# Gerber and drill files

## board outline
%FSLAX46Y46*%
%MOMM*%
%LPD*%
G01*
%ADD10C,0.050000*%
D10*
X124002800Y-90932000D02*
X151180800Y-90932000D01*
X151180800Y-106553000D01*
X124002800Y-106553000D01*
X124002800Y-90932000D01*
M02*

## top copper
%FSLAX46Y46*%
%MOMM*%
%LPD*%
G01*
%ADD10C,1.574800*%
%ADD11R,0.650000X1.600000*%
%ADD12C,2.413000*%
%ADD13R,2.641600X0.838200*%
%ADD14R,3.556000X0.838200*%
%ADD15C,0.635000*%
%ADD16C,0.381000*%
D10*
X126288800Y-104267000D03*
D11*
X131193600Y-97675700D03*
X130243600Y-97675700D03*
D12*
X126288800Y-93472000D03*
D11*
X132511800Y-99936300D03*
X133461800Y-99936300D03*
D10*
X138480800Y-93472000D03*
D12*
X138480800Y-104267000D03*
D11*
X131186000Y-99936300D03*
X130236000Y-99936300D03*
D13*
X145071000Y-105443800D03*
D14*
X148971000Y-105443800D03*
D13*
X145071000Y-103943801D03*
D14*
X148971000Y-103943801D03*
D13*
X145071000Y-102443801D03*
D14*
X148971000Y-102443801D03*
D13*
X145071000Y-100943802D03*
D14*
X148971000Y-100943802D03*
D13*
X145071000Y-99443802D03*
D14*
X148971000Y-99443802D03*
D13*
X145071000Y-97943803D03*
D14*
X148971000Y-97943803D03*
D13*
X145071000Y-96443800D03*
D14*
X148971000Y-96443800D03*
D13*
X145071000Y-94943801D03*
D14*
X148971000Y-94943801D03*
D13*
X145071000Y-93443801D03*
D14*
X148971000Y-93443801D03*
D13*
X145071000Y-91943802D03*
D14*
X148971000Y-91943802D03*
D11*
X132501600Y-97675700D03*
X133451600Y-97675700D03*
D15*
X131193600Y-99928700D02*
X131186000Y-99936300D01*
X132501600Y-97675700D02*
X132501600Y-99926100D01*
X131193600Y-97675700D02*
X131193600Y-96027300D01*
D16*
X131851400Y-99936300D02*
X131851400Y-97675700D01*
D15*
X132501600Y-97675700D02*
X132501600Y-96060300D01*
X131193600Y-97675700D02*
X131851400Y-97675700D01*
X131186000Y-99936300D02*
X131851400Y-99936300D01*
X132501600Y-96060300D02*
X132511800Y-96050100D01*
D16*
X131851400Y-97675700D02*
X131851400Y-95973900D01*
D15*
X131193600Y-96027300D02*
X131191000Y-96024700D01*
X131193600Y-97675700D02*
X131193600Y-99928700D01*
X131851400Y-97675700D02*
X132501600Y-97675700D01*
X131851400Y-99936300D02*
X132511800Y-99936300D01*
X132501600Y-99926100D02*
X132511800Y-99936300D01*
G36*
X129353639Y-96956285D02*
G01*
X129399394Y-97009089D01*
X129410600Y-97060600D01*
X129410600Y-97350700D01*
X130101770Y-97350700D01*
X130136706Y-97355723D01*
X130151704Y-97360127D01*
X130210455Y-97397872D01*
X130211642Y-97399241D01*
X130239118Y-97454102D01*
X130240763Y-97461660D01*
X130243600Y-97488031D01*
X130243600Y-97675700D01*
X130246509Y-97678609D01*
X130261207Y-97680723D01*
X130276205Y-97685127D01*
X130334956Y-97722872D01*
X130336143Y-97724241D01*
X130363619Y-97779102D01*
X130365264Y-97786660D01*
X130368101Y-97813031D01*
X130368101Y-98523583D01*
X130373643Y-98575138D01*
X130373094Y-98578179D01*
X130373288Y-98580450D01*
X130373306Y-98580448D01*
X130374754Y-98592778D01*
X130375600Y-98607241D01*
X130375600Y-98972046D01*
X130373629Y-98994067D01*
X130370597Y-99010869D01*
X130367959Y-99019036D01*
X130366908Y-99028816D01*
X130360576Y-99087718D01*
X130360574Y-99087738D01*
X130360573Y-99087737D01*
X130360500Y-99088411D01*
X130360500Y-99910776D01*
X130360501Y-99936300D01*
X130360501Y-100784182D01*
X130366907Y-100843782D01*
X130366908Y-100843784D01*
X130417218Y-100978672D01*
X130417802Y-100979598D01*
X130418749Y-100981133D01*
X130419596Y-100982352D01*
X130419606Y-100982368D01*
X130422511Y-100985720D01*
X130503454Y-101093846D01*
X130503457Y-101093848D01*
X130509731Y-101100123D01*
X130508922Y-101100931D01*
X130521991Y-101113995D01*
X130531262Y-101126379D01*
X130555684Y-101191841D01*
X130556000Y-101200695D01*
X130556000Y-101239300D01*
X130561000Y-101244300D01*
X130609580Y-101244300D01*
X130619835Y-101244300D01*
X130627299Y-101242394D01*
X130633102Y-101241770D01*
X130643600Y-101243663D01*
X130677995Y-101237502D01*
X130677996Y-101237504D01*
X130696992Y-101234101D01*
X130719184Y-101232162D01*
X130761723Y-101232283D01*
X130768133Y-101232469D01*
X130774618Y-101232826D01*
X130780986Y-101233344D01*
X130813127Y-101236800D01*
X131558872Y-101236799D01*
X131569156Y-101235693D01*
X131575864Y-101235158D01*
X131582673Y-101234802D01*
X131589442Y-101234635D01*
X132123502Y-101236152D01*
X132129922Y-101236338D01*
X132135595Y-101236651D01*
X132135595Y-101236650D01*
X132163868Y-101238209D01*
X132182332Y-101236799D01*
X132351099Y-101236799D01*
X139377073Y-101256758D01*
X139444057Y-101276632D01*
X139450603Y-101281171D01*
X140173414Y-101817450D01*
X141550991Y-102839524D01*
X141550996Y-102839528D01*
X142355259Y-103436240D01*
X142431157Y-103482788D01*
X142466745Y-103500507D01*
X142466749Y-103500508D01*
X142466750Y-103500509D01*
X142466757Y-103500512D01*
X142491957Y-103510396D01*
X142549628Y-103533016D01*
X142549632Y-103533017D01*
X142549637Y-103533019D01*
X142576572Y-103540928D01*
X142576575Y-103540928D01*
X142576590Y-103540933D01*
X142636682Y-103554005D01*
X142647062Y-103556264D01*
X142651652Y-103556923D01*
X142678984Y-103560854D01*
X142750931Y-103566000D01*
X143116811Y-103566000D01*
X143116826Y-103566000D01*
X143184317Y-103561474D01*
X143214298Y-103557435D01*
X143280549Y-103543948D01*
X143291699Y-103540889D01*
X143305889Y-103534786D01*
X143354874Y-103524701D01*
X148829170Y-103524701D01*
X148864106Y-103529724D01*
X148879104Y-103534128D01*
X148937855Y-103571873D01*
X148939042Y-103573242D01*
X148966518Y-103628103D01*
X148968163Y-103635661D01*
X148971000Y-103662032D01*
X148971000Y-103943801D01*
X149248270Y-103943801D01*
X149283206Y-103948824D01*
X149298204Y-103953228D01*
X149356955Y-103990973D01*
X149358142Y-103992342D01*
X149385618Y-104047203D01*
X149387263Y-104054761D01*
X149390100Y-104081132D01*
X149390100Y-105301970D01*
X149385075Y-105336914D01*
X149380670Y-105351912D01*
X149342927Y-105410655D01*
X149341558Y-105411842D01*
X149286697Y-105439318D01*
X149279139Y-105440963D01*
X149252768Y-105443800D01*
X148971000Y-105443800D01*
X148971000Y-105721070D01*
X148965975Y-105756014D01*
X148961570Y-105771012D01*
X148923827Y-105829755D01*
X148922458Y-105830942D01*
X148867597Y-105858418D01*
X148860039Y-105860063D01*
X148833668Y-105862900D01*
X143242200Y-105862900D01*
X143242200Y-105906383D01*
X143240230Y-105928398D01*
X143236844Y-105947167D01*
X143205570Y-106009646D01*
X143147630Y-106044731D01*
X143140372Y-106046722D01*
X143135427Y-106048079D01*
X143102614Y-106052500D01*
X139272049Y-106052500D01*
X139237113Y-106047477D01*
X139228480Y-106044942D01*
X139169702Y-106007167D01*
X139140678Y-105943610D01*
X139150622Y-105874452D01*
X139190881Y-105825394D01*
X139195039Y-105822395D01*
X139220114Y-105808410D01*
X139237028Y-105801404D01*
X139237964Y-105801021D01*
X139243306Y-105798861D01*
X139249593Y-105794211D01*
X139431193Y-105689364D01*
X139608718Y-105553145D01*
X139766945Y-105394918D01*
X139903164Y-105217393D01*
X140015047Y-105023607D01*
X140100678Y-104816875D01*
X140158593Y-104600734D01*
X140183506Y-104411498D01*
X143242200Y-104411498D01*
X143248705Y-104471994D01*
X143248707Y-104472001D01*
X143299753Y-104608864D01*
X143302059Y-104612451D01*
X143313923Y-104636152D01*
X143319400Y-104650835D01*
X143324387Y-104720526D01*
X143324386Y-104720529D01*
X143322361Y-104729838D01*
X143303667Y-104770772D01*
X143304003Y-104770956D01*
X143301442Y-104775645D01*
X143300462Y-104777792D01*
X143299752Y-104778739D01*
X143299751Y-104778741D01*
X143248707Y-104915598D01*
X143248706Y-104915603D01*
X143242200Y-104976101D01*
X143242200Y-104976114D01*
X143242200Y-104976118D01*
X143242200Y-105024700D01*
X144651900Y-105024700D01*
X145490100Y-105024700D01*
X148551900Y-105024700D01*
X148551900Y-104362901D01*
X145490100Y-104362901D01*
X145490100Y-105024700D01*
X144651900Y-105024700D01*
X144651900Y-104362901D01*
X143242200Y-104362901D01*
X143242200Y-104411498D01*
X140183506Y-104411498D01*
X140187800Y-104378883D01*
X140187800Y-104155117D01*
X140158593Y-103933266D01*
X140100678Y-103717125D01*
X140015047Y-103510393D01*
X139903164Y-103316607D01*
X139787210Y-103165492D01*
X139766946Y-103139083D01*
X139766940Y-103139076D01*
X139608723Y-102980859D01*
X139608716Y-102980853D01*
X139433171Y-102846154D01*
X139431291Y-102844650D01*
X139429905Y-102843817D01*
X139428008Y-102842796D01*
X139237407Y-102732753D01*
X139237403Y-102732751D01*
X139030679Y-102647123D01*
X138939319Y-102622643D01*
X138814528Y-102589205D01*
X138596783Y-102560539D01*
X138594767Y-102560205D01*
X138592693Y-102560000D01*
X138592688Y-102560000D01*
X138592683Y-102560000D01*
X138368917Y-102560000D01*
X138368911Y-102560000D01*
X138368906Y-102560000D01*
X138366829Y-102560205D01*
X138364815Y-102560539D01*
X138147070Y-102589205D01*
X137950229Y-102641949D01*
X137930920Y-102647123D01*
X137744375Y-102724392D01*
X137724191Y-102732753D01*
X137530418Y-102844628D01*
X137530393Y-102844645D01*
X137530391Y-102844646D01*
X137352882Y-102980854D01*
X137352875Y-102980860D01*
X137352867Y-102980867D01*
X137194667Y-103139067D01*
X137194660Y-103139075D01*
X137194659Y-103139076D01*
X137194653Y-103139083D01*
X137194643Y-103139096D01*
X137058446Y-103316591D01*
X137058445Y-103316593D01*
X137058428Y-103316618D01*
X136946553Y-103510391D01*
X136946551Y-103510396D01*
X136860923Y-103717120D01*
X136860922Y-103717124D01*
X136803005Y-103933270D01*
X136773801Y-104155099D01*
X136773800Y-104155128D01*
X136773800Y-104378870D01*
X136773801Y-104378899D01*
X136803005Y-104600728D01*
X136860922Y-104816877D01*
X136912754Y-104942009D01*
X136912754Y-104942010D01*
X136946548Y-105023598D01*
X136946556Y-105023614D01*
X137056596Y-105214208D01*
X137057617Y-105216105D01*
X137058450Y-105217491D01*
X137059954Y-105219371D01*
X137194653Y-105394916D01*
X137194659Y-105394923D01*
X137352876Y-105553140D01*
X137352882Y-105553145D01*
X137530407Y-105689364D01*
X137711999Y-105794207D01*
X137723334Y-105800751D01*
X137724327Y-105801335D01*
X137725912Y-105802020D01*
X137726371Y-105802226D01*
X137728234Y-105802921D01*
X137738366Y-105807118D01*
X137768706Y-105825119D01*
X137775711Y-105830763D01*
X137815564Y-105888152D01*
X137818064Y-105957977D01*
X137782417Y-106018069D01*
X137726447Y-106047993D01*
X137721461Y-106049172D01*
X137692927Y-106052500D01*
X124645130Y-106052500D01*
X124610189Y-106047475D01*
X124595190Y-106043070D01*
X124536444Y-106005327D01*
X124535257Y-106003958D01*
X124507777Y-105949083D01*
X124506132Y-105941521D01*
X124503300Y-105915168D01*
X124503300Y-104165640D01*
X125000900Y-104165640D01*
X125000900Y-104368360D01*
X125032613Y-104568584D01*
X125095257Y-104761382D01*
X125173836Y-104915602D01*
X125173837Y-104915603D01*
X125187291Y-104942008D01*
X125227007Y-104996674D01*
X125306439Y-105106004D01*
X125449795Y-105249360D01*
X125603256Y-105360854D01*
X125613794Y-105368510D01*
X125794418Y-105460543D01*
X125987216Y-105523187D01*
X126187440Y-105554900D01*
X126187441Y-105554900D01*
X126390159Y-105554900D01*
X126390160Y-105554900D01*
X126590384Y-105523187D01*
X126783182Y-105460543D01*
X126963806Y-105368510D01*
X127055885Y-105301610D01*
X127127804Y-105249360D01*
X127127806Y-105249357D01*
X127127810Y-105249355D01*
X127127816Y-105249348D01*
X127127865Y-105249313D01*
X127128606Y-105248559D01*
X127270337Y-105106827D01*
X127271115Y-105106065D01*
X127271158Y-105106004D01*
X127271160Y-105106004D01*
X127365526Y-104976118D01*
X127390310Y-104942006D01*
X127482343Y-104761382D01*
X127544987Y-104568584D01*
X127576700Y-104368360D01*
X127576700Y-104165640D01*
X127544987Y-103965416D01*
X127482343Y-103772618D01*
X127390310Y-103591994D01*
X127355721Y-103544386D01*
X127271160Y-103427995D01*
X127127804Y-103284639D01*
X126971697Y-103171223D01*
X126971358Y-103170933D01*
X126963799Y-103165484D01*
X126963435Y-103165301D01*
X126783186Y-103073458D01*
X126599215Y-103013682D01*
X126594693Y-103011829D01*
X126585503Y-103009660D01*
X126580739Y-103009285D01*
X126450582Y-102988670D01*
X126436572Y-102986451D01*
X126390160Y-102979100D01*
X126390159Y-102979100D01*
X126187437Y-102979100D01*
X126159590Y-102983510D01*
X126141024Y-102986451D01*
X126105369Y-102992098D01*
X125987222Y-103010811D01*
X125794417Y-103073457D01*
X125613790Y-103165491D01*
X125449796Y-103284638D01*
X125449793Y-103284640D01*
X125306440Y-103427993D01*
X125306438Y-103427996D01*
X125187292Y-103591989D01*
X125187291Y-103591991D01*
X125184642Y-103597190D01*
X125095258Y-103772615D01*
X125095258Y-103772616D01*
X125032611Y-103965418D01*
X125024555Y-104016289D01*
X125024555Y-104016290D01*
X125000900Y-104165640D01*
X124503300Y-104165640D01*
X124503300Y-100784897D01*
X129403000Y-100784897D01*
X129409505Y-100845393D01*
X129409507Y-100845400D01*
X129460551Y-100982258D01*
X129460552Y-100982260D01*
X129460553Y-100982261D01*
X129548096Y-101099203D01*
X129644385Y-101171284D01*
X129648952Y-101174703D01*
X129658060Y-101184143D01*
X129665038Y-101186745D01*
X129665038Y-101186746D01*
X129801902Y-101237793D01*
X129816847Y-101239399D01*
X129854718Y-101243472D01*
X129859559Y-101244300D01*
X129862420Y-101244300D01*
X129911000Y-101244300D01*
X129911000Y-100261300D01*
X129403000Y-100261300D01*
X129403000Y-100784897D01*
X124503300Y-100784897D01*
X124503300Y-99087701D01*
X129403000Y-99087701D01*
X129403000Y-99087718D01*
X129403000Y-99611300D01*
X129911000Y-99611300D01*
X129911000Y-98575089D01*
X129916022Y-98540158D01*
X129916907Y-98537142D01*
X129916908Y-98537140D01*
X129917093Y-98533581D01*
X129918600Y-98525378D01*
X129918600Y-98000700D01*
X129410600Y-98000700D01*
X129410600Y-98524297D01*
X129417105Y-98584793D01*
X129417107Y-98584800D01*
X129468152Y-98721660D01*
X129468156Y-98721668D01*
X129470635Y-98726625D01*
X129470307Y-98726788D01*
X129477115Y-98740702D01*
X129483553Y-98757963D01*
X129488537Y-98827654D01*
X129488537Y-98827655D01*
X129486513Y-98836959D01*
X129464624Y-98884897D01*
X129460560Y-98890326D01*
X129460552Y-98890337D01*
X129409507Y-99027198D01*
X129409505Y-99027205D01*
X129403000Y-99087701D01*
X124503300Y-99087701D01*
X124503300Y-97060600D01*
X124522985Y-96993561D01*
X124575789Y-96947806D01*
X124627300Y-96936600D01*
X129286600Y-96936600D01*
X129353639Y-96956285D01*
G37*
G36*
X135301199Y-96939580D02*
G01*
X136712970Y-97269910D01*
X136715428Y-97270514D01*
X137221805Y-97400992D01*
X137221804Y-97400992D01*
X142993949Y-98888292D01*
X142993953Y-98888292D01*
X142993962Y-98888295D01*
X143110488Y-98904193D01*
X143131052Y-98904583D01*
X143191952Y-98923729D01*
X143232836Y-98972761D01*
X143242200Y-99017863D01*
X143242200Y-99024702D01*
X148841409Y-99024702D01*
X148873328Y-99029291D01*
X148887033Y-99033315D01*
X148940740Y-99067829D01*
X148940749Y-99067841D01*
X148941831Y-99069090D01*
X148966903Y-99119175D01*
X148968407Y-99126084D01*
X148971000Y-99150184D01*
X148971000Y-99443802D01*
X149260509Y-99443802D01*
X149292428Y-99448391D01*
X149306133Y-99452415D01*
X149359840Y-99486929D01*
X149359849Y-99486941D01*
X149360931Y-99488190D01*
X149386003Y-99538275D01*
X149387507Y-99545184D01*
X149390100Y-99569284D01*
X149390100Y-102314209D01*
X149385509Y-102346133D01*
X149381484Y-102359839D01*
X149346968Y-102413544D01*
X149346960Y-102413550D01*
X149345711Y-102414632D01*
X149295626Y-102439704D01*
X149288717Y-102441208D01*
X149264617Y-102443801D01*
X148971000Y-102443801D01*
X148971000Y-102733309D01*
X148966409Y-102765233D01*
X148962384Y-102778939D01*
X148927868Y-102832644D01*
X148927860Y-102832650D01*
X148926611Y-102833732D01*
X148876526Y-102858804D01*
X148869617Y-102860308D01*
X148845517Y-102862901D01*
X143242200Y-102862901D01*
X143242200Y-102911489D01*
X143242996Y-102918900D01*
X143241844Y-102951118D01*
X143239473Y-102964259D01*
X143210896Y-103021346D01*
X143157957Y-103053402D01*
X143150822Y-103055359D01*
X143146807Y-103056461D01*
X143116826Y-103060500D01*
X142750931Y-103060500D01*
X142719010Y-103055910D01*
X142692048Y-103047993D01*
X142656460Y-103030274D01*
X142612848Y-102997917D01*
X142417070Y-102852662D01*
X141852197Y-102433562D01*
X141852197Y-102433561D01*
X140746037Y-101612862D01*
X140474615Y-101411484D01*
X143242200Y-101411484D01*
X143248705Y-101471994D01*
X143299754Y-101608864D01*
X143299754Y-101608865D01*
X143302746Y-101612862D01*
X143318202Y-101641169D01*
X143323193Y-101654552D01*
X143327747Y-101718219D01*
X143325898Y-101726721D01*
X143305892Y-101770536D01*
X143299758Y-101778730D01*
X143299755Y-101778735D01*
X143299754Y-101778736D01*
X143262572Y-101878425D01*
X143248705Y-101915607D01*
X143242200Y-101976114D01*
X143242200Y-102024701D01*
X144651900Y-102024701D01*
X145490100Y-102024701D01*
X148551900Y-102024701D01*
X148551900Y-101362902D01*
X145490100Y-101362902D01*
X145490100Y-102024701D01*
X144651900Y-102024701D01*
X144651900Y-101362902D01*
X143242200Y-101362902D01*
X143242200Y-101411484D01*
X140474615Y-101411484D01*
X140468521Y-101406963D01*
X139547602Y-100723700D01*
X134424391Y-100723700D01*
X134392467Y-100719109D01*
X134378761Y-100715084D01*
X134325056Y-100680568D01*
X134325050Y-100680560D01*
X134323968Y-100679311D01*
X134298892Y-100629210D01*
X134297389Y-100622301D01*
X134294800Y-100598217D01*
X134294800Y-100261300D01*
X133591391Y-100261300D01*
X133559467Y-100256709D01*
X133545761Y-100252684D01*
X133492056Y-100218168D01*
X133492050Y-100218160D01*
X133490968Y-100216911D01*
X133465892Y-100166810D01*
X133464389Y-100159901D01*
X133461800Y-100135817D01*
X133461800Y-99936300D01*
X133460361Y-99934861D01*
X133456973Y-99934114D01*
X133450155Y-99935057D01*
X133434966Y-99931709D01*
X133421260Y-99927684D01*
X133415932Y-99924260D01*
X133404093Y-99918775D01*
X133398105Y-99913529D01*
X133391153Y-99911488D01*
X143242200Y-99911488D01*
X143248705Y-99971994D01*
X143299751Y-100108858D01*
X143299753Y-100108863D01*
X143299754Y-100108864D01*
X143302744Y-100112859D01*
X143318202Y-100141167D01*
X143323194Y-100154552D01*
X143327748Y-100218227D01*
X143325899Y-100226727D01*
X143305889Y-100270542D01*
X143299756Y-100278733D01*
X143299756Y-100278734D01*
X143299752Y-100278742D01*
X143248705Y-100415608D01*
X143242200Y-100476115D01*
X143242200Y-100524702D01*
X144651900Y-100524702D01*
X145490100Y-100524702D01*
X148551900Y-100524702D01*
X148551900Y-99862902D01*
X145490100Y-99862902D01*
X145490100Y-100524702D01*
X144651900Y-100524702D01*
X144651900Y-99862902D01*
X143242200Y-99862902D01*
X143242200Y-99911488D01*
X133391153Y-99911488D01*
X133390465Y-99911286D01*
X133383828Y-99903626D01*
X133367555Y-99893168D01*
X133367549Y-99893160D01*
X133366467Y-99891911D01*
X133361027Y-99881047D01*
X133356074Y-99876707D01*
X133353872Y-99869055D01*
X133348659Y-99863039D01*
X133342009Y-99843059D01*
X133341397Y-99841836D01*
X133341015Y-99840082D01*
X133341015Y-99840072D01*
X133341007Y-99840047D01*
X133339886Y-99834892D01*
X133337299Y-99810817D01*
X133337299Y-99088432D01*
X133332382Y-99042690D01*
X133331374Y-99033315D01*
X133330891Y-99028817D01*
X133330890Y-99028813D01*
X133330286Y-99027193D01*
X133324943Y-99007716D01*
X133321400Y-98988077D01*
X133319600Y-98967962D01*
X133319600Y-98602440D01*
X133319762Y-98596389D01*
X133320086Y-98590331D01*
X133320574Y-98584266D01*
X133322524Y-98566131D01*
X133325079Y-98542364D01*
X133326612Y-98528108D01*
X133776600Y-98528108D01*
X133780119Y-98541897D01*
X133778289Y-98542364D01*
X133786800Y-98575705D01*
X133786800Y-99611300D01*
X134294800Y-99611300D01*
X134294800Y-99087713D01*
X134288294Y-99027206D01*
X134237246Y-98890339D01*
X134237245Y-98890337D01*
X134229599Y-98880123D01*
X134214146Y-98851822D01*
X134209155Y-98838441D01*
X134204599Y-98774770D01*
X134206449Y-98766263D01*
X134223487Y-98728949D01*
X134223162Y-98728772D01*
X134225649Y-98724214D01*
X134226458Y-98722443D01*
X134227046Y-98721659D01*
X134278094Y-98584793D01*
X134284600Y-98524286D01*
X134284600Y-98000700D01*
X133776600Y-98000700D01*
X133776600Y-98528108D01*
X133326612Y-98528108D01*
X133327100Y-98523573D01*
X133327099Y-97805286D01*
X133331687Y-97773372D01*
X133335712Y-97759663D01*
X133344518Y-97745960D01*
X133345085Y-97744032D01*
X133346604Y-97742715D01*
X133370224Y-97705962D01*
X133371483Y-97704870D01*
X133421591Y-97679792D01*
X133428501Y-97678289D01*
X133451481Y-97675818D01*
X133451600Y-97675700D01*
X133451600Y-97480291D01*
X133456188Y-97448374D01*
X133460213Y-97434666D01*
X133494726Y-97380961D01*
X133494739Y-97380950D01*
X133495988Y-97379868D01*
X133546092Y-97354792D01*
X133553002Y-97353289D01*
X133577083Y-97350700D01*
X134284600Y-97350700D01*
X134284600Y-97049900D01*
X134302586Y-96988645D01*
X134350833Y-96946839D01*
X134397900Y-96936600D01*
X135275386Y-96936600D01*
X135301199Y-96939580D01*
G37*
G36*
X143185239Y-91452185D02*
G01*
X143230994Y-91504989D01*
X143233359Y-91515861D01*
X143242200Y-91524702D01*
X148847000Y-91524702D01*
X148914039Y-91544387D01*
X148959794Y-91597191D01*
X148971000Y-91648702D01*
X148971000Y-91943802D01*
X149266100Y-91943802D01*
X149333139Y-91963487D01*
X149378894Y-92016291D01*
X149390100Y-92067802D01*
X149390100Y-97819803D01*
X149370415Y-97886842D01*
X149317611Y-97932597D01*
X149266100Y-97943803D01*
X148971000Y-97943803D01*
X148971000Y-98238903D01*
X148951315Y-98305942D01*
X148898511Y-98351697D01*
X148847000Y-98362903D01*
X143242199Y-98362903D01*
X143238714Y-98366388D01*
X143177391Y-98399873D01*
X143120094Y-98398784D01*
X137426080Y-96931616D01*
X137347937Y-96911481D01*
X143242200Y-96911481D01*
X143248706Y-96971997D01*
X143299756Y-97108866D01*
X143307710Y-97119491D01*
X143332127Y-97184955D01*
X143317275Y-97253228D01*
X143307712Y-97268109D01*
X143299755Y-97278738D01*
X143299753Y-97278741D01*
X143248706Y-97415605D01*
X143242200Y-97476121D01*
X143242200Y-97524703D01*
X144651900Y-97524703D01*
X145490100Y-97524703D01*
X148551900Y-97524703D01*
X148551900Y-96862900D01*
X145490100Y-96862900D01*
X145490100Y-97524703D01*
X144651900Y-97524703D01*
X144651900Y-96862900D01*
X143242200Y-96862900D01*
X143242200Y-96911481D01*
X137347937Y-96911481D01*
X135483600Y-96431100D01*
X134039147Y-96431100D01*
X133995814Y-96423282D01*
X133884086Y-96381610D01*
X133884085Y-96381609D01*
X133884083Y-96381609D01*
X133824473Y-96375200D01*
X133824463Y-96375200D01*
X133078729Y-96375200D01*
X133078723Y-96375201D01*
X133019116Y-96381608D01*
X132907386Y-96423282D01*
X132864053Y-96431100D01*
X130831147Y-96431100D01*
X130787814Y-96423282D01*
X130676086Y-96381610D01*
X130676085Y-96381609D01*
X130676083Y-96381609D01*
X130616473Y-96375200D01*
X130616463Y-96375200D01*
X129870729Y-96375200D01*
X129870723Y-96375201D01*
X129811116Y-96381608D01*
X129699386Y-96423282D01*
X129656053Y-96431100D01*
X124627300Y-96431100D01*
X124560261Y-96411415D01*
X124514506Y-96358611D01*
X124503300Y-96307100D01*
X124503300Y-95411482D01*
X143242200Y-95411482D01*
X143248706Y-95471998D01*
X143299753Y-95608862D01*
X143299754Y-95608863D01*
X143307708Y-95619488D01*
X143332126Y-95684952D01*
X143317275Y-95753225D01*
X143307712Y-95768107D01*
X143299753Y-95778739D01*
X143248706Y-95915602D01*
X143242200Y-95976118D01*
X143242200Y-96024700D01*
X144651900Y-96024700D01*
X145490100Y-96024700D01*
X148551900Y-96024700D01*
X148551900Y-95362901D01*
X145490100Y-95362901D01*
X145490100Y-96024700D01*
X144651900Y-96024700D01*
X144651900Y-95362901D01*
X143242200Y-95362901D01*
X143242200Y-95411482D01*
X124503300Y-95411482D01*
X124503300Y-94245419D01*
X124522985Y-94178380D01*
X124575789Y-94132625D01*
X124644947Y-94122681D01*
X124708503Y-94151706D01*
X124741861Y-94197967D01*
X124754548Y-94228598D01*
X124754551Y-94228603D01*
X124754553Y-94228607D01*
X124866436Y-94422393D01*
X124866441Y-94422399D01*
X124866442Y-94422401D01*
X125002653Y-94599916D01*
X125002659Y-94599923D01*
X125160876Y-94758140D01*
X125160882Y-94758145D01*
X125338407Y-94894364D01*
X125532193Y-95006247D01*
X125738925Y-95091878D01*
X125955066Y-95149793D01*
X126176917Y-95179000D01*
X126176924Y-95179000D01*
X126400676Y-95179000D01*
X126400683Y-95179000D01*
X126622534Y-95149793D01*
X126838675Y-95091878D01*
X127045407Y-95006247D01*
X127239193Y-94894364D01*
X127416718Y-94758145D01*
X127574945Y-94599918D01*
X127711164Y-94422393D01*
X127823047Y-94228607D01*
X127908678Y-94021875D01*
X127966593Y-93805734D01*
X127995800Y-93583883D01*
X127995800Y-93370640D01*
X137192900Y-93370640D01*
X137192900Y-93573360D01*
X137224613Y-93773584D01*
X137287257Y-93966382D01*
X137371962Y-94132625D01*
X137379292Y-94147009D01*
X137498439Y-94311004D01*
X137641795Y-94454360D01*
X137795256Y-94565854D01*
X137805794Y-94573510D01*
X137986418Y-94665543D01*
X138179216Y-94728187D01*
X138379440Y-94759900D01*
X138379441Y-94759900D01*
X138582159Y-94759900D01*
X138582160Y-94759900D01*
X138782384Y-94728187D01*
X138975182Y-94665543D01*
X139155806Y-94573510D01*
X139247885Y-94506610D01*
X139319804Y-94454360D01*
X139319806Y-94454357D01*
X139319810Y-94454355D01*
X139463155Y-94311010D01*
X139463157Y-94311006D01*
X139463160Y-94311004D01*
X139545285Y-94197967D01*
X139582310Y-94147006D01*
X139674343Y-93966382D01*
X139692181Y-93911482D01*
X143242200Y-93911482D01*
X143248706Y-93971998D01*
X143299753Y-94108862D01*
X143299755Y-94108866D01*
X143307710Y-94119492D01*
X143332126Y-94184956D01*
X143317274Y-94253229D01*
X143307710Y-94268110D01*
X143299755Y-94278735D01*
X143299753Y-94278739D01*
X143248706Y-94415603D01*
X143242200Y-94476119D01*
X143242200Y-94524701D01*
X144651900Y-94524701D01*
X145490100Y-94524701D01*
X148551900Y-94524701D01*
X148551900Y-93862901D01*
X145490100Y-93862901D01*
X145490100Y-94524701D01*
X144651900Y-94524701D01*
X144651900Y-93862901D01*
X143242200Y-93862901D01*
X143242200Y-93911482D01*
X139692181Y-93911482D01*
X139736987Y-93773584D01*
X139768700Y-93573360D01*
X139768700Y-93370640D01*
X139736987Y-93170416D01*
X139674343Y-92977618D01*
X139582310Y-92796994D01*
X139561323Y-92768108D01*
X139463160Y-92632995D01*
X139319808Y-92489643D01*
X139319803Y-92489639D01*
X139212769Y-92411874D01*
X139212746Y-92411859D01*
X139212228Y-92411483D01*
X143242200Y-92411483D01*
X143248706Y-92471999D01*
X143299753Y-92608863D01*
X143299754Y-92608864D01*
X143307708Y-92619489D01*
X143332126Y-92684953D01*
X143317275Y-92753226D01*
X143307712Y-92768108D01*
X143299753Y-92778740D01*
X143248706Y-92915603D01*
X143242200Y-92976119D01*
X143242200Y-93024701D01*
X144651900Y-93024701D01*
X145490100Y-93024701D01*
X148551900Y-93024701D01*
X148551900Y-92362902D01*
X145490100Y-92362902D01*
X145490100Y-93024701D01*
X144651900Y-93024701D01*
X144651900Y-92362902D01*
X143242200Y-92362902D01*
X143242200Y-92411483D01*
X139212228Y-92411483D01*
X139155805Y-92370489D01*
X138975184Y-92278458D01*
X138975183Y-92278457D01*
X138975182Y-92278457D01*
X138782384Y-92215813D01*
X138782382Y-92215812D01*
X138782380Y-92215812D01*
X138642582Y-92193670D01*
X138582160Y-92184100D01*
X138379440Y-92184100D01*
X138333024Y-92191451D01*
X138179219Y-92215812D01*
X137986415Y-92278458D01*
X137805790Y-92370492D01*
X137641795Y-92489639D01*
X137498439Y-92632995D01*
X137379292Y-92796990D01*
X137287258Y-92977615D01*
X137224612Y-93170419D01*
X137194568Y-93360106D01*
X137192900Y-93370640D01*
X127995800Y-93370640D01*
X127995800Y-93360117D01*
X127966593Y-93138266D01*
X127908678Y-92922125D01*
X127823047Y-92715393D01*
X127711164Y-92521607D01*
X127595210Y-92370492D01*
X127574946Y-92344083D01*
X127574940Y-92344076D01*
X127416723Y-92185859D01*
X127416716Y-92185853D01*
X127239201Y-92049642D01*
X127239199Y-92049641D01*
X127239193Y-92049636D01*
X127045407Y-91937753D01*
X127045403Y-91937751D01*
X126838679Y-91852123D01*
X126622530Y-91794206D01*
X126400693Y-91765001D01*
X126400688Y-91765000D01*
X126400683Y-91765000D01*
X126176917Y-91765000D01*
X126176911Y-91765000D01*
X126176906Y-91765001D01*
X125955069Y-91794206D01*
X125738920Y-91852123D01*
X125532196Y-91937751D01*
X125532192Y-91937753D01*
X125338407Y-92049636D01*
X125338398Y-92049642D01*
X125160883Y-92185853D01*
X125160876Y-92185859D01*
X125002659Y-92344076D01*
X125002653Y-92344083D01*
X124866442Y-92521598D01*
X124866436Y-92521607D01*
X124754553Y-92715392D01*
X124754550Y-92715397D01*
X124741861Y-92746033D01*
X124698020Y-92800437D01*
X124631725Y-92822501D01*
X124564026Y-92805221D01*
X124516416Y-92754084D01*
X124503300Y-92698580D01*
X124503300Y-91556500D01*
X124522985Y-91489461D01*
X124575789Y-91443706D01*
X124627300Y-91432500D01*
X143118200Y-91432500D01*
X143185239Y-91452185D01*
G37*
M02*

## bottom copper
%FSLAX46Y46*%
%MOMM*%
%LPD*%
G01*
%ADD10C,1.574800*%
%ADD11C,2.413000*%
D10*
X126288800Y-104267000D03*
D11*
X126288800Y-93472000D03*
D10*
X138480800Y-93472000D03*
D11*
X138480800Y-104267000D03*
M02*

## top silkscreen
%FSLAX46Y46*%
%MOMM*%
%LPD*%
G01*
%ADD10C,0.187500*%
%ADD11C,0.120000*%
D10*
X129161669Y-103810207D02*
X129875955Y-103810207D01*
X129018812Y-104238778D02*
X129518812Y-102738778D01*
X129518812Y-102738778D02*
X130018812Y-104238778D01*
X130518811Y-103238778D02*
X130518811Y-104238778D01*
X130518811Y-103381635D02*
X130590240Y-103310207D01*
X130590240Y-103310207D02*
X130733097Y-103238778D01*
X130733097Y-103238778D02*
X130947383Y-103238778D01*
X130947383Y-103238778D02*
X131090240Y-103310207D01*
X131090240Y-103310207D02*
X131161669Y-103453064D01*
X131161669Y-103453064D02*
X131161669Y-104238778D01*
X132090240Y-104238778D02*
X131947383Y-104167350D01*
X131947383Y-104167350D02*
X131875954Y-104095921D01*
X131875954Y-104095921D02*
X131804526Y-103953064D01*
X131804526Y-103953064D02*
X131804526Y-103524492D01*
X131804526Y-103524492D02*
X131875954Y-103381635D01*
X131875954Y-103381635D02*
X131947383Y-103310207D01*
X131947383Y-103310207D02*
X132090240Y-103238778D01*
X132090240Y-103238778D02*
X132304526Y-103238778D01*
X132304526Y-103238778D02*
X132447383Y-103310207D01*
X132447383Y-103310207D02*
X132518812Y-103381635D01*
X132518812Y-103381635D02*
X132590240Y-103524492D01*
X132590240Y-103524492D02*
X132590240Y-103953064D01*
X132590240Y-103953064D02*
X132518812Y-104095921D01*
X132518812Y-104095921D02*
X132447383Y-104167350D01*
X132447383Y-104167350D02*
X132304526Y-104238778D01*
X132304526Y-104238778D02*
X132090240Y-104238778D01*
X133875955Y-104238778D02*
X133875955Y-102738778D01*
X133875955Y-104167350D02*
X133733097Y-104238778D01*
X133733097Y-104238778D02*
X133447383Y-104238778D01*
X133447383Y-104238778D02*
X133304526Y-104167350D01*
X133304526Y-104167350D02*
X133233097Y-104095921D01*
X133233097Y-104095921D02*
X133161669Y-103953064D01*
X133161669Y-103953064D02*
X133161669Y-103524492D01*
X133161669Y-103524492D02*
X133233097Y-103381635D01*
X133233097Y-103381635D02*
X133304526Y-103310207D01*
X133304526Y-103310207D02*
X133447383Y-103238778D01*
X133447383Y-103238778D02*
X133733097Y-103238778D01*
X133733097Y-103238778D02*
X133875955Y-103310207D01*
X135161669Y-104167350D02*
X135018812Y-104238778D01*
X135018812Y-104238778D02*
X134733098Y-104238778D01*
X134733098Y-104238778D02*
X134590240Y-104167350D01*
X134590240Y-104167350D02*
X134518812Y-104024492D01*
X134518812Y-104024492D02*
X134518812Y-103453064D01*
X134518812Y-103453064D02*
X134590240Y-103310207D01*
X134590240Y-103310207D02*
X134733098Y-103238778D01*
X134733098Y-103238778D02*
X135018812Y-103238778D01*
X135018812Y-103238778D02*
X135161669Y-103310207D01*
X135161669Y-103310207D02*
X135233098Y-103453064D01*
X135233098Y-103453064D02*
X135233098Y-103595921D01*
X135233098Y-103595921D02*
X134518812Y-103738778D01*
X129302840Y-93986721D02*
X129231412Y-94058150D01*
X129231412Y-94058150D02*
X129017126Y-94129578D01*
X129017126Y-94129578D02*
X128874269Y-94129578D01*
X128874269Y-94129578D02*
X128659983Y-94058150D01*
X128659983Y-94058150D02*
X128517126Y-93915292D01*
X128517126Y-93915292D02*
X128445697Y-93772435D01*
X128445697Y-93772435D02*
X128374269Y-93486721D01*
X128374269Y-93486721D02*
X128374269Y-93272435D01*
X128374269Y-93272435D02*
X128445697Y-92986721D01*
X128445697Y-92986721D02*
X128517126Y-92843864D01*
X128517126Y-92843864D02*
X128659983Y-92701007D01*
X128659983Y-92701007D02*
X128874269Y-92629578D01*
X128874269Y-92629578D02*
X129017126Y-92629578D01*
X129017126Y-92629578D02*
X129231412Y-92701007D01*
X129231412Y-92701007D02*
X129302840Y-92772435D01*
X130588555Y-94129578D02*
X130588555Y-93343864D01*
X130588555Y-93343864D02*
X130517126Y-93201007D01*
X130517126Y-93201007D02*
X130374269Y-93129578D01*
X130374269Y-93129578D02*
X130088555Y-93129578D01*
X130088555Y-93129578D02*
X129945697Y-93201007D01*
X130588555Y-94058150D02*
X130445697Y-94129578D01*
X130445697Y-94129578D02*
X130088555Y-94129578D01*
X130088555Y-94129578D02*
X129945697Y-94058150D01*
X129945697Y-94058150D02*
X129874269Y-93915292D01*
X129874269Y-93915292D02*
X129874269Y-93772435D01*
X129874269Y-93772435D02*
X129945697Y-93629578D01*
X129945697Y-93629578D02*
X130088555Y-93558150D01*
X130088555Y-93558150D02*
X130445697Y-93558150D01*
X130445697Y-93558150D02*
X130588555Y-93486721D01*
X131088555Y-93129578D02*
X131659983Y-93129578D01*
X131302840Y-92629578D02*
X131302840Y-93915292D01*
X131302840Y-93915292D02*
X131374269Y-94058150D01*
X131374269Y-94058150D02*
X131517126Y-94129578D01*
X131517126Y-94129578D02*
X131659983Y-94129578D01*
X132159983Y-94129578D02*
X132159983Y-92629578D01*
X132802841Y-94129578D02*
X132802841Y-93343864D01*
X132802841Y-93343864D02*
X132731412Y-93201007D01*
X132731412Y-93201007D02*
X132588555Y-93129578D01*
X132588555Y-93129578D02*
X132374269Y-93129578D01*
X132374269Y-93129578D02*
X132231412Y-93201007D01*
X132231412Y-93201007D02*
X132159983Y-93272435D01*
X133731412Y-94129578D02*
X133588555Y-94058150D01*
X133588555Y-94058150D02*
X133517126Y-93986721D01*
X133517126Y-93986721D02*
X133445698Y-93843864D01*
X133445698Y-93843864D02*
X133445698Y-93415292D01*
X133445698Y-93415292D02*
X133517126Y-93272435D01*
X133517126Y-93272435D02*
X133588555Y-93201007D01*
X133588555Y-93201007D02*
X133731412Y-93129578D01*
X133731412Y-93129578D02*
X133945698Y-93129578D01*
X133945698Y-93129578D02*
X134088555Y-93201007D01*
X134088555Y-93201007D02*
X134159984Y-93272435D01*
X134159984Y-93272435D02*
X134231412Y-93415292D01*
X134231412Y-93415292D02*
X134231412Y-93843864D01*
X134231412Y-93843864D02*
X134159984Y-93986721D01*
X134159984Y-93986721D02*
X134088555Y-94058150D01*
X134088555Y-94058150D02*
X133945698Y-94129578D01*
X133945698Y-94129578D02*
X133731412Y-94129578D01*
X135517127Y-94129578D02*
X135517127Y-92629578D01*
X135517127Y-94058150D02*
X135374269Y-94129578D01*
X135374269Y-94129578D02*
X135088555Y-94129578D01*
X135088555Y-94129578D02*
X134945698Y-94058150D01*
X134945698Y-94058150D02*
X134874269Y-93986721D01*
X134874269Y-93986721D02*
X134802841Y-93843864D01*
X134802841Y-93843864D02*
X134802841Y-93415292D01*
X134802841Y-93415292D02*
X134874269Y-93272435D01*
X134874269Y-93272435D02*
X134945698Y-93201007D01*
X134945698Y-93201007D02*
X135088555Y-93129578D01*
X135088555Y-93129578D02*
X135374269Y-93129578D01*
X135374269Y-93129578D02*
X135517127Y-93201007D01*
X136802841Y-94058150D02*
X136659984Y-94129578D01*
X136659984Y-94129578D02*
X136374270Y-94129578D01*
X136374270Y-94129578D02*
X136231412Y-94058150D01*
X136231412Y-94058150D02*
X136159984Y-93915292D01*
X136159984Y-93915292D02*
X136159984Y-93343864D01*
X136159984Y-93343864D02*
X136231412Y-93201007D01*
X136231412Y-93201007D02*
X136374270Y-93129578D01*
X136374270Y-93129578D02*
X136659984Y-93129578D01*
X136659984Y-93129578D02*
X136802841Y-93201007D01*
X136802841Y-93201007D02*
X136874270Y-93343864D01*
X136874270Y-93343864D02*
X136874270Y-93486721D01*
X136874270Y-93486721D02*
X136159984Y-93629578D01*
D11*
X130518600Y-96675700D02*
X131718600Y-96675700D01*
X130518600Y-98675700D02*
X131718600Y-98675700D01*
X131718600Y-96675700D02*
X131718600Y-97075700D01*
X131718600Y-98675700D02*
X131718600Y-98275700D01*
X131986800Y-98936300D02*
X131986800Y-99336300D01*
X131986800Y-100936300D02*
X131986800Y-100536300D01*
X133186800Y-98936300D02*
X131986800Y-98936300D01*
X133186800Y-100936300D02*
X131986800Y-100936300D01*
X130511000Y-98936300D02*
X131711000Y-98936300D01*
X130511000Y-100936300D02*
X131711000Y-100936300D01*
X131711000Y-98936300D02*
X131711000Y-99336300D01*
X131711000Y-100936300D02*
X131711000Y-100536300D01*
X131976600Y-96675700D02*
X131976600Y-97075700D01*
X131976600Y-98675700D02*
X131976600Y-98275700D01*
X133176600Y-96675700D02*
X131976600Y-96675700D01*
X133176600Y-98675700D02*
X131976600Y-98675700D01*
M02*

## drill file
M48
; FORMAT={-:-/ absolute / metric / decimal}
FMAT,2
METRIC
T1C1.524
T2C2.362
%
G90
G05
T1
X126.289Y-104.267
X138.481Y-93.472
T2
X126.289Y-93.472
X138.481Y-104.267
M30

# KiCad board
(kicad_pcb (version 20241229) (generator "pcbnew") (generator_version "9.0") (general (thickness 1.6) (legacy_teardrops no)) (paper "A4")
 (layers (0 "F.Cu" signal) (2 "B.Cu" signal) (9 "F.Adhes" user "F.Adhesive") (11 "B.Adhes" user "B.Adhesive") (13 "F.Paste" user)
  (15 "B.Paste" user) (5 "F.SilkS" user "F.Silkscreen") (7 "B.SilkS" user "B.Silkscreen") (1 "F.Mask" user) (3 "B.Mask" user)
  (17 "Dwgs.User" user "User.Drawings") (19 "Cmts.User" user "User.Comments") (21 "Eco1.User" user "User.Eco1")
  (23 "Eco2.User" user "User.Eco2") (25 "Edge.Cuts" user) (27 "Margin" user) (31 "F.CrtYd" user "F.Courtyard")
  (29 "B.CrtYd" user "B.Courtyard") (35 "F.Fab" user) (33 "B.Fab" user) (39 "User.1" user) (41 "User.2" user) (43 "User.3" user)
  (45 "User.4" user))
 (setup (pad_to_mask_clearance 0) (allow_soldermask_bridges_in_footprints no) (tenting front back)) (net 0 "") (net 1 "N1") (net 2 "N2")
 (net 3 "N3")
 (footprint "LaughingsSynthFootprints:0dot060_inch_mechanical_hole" (layer "F.Cu") (at 126.2888 104.267)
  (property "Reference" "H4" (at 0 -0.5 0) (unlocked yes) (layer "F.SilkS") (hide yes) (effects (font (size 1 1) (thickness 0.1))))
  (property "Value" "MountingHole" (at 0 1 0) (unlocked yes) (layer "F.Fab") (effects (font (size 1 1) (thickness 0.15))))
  (pad "" np_thru_hole circle (at 0 0) (size 1.5748 1.5748) (drill 1.524) (layers "*.Cu" "*.Mask")))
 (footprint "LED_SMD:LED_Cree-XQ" (layer "F.Cu") (at 130.7186 97.6757 180)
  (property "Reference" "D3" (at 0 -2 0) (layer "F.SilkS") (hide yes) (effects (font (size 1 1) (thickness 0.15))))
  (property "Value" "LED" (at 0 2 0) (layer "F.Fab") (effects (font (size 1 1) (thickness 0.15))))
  (fp_line (start 0.2 1) (end -1 1) (stroke (width 0.12) (type solid)) (layer "F.SilkS"))
  (fp_line (start 0.2 -1) (end -1 -1) (stroke (width 0.12) (type solid)) (layer "F.SilkS"))
  (fp_line (start -1 1) (end -1 0.6) (stroke (width 0.12) (type solid)) (layer "F.SilkS"))
  (fp_line (start -1 -1) (end -1 -0.6) (stroke (width 0.12) (type solid)) (layer "F.SilkS"))
  (pad "1" smd rect (at -0.475 0 180) (size 0.65 1.6) (layers "F.Cu" "F.Mask" "F.Paste") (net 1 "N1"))
  (pad "2" smd rect (at 0.475 0 180) (size 0.65 1.6) (layers "F.Cu" "F.Mask" "F.Paste") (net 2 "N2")))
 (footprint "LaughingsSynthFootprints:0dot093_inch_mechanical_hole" (layer "F.Cu") (at 126.2888 93.472)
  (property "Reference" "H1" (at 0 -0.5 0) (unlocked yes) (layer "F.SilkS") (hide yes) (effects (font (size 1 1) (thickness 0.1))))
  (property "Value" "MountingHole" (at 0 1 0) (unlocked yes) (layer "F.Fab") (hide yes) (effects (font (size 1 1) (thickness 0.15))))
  (pad "" np_thru_hole circle (at 0 0) (size 2.413 2.413) (drill 2.3622) (layers "*.Cu" "*.Mask")))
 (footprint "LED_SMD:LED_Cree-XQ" (layer "F.Cu") (at 132.9868 99.9363)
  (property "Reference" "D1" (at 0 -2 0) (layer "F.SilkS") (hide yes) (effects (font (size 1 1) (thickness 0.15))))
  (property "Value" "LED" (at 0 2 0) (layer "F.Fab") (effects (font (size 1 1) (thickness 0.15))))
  (fp_line (start -1 -1) (end -1 -0.6) (stroke (width 0.12) (type solid)) (layer "F.SilkS"))
  (fp_line (start -1 1) (end -1 0.6) (stroke (width 0.12) (type solid)) (layer "F.SilkS"))
  (fp_line (start 0.2 -1) (end -1 -1) (stroke (width 0.12) (type solid)) (layer "F.SilkS"))
  (fp_line (start 0.2 1) (end -1 1) (stroke (width 0.12) (type solid)) (layer "F.SilkS"))
  (pad "1" smd rect (at -0.475 0) (size 0.65 1.6) (layers "F.Cu" "F.Mask" "F.Paste") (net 1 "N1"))
  (pad "2" smd rect (at 0.475 0) (size 0.65 1.6) (layers "F.Cu" "F.Mask" "F.Paste") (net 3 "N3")))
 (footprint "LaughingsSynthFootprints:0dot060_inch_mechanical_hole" (layer "F.Cu") (at 138.4808 93.472)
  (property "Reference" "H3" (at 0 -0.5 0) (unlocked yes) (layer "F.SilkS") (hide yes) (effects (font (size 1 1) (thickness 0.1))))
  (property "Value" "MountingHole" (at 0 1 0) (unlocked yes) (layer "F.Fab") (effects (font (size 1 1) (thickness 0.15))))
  (pad "" np_thru_hole circle (at 0 0) (size 1.5748 1.5748) (drill 1.524) (layers "*.Cu" "*.Mask")))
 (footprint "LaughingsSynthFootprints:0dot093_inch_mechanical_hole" (layer "F.Cu") (at 138.4808 104.267)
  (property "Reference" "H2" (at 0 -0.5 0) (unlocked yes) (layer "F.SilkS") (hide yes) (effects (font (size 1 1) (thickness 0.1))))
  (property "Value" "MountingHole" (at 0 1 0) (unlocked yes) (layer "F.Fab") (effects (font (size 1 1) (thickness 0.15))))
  (pad "" np_thru_hole circle (at 0 0) (size 2.413 2.413) (drill 2.3622) (layers "*.Cu" "*.Mask")))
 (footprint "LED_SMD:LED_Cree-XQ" (layer "F.Cu") (at 130.711 99.9363 180)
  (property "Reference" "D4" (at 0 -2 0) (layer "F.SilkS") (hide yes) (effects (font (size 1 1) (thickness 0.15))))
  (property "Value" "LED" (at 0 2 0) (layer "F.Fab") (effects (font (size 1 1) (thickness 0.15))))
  (fp_line (start 0.2 1) (end -1 1) (stroke (width 0.12) (type solid)) (layer "F.SilkS"))
  (fp_line (start 0.2 -1) (end -1 -1) (stroke (width 0.12) (type solid)) (layer "F.SilkS"))
  (fp_line (start -1 1) (end -1 0.6) (stroke (width 0.12) (type solid)) (layer "F.SilkS"))
  (fp_line (start -1 -1) (end -1 -0.6) (stroke (width 0.12) (type solid)) (layer "F.SilkS"))
  (pad "1" smd rect (at -0.475 0 180) (size 0.65 1.6) (layers "F.Cu" "F.Mask" "F.Paste") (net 1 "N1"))
  (pad "2" smd rect (at 0.475 0 180) (size 0.65 1.6) (layers "F.Cu" "F.Mask" "F.Paste") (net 2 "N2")))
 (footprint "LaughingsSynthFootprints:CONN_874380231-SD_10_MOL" (layer "F.Cu") (at 149.116199 98.693801 90)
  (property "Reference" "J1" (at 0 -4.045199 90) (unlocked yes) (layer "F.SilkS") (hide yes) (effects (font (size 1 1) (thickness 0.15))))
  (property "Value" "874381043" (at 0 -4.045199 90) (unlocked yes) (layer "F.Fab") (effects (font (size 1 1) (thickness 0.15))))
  (pad "1_1" smd rect (at -6.749999 -4.045199 90) (size 0.8382 2.6416) (layers "F.Cu" "F.Mask" "F.Paste") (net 2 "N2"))
  (pad "1_2" smd rect (at -6.749999 -0.145199 90) (size 0.8382 3.556) (layers "F.Cu" "F.Mask" "F.Paste") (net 2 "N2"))
  (pad "2_1" smd rect (at -5.25 -4.045199 90) (size 0.8382 2.6416) (layers "F.Cu" "F.Mask" "F.Paste") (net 2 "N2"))
  (pad "2_2" smd rect (at -5.25 -0.145199 90) (size 0.8382 3.556) (layers "F.Cu" "F.Mask" "F.Paste") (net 2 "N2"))
  (pad "3_1" smd rect (at -3.75 -4.045199 90) (size 0.8382 2.6416) (layers "F.Cu" "F.Mask" "F.Paste") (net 3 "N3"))
  (pad "3_2" smd rect (at -3.75 -0.145199 90) (size 0.8382 3.556) (layers "F.Cu" "F.Mask" "F.Paste") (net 3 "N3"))
  (pad "4_1" smd rect (at -2.250001 -4.045199 90) (size 0.8382 2.6416) (layers "F.Cu" "F.Mask" "F.Paste") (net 3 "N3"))
  (pad "4_2" smd rect (at -2.250001 -0.145199 90) (size 0.8382 3.556) (layers "F.Cu" "F.Mask" "F.Paste") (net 3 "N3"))
  (pad "5_1" smd rect (at -0.750001 -4.045199 90) (size 0.8382 2.6416) (layers "F.Cu" "F.Mask" "F.Paste") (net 3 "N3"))
  (pad "5_2" smd rect (at -0.750001 -0.145199 90) (size 0.8382 3.556) (layers "F.Cu" "F.Mask" "F.Paste") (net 3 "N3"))
  (pad "6_1" smd rect (at 0.749998 -4.045199 90) (size 0.8382 2.6416) (layers "F.Cu" "F.Mask" "F.Paste") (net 1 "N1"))
  (pad "6_2" smd rect (at 0.749998 -0.145199 90) (size 0.8382 3.556) (layers "F.Cu" "F.Mask" "F.Paste") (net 1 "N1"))
  (pad "7_1" smd rect (at 2.250001 -4.045199 90) (size 0.8382 2.6416) (layers "F.Cu" "F.Mask" "F.Paste") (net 1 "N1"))
  (pad "7_2" smd rect (at 2.250001 -0.145199 90) (size 0.8382 3.556) (layers "F.Cu" "F.Mask" "F.Paste") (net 1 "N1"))
  (pad "8_1" smd rect (at 3.75 -4.045199 90) (size 0.8382 2.6416) (layers "F.Cu" "F.Mask" "F.Paste") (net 1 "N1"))
  (pad "8_2" smd rect (at 3.75 -0.145199 90) (size 0.8382 3.556) (layers "F.Cu" "F.Mask" "F.Paste") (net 1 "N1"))
  (pad "9_1" smd rect (at 5.25 -4.045199 90) (size 0.8382 2.6416) (layers "F.Cu" "F.Mask" "F.Paste") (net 1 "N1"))
  (pad "9_2" smd rect (at 5.25 -0.145199 90) (size 0.8382 3.556) (layers "F.Cu" "F.Mask" "F.Paste") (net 1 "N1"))
  (pad "10_1" smd rect (at 6.749999 -4.045199 90) (size 0.8382 2.6416) (layers "F.Cu" "F.Mask" "F.Paste") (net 1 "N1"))
  (pad "10_2" smd rect (at 6.749999 -0.145199 90) (size 0.8382 3.556) (layers "F.Cu" "F.Mask" "F.Paste") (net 1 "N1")))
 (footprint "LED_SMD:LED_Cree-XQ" (layer "F.Cu") (at 132.9766 97.6757)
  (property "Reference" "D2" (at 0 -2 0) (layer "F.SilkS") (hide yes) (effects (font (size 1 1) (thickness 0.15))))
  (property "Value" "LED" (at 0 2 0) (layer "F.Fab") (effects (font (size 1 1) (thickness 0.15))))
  (fp_line (start -1 -1) (end -1 -0.6) (stroke (width 0.12) (type solid)) (layer "F.SilkS"))
  (fp_line (start -1 1) (end -1 0.6) (stroke (width 0.12) (type solid)) (layer "F.SilkS"))
  (fp_line (start 0.2 -1) (end -1 -1) (stroke (width 0.12) (type solid)) (layer "F.SilkS"))
  (fp_line (start 0.2 1) (end -1 1) (stroke (width 0.12) (type solid)) (layer "F.SilkS"))
  (pad "1" smd rect (at -0.475 0) (size 0.65 1.6) (layers "F.Cu" "F.Mask" "F.Paste") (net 1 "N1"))
  (pad "2" smd rect (at 0.475 0) (size 0.65 1.6) (layers "F.Cu" "F.Mask" "F.Paste") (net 3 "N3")))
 (gr_rect (start 124.0028 90.932) (end 151.1808 106.553) (stroke (width 0.05) (type default)) (fill no) (layer "Edge.Cuts"))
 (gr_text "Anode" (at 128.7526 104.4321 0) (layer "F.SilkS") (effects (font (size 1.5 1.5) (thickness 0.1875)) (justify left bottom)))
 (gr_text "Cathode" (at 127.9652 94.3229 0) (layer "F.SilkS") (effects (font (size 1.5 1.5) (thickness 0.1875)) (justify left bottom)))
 (segment (start 131.1936 99.9287) (end 131.186 99.9363) (width 0.635) (layer "F.Cu") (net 1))
 (segment (start 132.5016 97.6757) (end 132.5016 99.9261) (width 0.635) (layer "F.Cu") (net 1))
 (segment (start 131.1936 97.6757) (end 131.1936 96.0273) (width 0.635) (layer "F.Cu") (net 1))
 (segment (start 131.8514 99.9363) (end 131.8514 97.6757) (width 0.381) (layer "F.Cu") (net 1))
 (segment (start 132.5016 97.6757) (end 132.5016 96.0603) (width 0.635) (layer "F.Cu") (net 1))
 (segment (start 131.1936 97.6757) (end 131.8514 97.6757) (width 0.635) (layer "F.Cu") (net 1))
 (segment (start 131.186 99.9363) (end 131.8514 99.9363) (width 0.635) (layer "F.Cu") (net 1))
 (segment (start 132.5016 96.0603) (end 132.5118 96.0501) (width 0.635) (layer "F.Cu") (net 1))
 (segment (start 131.8514 97.6757) (end 131.8514 95.9739) (width 0.381) (layer "F.Cu") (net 1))
 (segment (start 131.1936 96.0273) (end 131.191 96.0247) (width 0.635) (layer "F.Cu") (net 1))
 (segment (start 131.1936 97.6757) (end 131.1936 99.9287) (width 0.635) (layer "F.Cu") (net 1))
 (segment (start 131.8514 97.6757) (end 132.5016 97.6757) (width 0.635) (layer "F.Cu") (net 1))
 (segment (start 131.8514 99.9363) (end 132.5118 99.9363) (width 0.635) (layer "F.Cu") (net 1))
 (segment (start 132.5016 99.9261) (end 132.5118 99.9363) (width 0.635) (layer "F.Cu") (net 1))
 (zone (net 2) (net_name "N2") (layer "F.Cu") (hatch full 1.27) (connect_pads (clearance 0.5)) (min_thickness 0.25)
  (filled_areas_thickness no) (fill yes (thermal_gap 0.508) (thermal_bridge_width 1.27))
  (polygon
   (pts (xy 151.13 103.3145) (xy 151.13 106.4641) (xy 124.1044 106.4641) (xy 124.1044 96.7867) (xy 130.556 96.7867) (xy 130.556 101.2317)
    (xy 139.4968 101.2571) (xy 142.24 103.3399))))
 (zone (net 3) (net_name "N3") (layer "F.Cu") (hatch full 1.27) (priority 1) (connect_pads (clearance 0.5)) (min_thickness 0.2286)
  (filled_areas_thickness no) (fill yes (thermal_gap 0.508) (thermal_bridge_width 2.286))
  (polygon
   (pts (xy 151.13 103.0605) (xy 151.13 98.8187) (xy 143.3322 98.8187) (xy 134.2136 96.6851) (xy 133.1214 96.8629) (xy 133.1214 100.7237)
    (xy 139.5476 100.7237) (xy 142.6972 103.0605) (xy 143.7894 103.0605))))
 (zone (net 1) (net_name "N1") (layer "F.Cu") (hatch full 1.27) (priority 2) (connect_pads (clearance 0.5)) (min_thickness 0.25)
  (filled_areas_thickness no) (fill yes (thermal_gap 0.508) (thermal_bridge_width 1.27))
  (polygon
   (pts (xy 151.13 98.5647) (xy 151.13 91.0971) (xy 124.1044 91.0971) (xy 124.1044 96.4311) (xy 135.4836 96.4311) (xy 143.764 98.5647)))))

